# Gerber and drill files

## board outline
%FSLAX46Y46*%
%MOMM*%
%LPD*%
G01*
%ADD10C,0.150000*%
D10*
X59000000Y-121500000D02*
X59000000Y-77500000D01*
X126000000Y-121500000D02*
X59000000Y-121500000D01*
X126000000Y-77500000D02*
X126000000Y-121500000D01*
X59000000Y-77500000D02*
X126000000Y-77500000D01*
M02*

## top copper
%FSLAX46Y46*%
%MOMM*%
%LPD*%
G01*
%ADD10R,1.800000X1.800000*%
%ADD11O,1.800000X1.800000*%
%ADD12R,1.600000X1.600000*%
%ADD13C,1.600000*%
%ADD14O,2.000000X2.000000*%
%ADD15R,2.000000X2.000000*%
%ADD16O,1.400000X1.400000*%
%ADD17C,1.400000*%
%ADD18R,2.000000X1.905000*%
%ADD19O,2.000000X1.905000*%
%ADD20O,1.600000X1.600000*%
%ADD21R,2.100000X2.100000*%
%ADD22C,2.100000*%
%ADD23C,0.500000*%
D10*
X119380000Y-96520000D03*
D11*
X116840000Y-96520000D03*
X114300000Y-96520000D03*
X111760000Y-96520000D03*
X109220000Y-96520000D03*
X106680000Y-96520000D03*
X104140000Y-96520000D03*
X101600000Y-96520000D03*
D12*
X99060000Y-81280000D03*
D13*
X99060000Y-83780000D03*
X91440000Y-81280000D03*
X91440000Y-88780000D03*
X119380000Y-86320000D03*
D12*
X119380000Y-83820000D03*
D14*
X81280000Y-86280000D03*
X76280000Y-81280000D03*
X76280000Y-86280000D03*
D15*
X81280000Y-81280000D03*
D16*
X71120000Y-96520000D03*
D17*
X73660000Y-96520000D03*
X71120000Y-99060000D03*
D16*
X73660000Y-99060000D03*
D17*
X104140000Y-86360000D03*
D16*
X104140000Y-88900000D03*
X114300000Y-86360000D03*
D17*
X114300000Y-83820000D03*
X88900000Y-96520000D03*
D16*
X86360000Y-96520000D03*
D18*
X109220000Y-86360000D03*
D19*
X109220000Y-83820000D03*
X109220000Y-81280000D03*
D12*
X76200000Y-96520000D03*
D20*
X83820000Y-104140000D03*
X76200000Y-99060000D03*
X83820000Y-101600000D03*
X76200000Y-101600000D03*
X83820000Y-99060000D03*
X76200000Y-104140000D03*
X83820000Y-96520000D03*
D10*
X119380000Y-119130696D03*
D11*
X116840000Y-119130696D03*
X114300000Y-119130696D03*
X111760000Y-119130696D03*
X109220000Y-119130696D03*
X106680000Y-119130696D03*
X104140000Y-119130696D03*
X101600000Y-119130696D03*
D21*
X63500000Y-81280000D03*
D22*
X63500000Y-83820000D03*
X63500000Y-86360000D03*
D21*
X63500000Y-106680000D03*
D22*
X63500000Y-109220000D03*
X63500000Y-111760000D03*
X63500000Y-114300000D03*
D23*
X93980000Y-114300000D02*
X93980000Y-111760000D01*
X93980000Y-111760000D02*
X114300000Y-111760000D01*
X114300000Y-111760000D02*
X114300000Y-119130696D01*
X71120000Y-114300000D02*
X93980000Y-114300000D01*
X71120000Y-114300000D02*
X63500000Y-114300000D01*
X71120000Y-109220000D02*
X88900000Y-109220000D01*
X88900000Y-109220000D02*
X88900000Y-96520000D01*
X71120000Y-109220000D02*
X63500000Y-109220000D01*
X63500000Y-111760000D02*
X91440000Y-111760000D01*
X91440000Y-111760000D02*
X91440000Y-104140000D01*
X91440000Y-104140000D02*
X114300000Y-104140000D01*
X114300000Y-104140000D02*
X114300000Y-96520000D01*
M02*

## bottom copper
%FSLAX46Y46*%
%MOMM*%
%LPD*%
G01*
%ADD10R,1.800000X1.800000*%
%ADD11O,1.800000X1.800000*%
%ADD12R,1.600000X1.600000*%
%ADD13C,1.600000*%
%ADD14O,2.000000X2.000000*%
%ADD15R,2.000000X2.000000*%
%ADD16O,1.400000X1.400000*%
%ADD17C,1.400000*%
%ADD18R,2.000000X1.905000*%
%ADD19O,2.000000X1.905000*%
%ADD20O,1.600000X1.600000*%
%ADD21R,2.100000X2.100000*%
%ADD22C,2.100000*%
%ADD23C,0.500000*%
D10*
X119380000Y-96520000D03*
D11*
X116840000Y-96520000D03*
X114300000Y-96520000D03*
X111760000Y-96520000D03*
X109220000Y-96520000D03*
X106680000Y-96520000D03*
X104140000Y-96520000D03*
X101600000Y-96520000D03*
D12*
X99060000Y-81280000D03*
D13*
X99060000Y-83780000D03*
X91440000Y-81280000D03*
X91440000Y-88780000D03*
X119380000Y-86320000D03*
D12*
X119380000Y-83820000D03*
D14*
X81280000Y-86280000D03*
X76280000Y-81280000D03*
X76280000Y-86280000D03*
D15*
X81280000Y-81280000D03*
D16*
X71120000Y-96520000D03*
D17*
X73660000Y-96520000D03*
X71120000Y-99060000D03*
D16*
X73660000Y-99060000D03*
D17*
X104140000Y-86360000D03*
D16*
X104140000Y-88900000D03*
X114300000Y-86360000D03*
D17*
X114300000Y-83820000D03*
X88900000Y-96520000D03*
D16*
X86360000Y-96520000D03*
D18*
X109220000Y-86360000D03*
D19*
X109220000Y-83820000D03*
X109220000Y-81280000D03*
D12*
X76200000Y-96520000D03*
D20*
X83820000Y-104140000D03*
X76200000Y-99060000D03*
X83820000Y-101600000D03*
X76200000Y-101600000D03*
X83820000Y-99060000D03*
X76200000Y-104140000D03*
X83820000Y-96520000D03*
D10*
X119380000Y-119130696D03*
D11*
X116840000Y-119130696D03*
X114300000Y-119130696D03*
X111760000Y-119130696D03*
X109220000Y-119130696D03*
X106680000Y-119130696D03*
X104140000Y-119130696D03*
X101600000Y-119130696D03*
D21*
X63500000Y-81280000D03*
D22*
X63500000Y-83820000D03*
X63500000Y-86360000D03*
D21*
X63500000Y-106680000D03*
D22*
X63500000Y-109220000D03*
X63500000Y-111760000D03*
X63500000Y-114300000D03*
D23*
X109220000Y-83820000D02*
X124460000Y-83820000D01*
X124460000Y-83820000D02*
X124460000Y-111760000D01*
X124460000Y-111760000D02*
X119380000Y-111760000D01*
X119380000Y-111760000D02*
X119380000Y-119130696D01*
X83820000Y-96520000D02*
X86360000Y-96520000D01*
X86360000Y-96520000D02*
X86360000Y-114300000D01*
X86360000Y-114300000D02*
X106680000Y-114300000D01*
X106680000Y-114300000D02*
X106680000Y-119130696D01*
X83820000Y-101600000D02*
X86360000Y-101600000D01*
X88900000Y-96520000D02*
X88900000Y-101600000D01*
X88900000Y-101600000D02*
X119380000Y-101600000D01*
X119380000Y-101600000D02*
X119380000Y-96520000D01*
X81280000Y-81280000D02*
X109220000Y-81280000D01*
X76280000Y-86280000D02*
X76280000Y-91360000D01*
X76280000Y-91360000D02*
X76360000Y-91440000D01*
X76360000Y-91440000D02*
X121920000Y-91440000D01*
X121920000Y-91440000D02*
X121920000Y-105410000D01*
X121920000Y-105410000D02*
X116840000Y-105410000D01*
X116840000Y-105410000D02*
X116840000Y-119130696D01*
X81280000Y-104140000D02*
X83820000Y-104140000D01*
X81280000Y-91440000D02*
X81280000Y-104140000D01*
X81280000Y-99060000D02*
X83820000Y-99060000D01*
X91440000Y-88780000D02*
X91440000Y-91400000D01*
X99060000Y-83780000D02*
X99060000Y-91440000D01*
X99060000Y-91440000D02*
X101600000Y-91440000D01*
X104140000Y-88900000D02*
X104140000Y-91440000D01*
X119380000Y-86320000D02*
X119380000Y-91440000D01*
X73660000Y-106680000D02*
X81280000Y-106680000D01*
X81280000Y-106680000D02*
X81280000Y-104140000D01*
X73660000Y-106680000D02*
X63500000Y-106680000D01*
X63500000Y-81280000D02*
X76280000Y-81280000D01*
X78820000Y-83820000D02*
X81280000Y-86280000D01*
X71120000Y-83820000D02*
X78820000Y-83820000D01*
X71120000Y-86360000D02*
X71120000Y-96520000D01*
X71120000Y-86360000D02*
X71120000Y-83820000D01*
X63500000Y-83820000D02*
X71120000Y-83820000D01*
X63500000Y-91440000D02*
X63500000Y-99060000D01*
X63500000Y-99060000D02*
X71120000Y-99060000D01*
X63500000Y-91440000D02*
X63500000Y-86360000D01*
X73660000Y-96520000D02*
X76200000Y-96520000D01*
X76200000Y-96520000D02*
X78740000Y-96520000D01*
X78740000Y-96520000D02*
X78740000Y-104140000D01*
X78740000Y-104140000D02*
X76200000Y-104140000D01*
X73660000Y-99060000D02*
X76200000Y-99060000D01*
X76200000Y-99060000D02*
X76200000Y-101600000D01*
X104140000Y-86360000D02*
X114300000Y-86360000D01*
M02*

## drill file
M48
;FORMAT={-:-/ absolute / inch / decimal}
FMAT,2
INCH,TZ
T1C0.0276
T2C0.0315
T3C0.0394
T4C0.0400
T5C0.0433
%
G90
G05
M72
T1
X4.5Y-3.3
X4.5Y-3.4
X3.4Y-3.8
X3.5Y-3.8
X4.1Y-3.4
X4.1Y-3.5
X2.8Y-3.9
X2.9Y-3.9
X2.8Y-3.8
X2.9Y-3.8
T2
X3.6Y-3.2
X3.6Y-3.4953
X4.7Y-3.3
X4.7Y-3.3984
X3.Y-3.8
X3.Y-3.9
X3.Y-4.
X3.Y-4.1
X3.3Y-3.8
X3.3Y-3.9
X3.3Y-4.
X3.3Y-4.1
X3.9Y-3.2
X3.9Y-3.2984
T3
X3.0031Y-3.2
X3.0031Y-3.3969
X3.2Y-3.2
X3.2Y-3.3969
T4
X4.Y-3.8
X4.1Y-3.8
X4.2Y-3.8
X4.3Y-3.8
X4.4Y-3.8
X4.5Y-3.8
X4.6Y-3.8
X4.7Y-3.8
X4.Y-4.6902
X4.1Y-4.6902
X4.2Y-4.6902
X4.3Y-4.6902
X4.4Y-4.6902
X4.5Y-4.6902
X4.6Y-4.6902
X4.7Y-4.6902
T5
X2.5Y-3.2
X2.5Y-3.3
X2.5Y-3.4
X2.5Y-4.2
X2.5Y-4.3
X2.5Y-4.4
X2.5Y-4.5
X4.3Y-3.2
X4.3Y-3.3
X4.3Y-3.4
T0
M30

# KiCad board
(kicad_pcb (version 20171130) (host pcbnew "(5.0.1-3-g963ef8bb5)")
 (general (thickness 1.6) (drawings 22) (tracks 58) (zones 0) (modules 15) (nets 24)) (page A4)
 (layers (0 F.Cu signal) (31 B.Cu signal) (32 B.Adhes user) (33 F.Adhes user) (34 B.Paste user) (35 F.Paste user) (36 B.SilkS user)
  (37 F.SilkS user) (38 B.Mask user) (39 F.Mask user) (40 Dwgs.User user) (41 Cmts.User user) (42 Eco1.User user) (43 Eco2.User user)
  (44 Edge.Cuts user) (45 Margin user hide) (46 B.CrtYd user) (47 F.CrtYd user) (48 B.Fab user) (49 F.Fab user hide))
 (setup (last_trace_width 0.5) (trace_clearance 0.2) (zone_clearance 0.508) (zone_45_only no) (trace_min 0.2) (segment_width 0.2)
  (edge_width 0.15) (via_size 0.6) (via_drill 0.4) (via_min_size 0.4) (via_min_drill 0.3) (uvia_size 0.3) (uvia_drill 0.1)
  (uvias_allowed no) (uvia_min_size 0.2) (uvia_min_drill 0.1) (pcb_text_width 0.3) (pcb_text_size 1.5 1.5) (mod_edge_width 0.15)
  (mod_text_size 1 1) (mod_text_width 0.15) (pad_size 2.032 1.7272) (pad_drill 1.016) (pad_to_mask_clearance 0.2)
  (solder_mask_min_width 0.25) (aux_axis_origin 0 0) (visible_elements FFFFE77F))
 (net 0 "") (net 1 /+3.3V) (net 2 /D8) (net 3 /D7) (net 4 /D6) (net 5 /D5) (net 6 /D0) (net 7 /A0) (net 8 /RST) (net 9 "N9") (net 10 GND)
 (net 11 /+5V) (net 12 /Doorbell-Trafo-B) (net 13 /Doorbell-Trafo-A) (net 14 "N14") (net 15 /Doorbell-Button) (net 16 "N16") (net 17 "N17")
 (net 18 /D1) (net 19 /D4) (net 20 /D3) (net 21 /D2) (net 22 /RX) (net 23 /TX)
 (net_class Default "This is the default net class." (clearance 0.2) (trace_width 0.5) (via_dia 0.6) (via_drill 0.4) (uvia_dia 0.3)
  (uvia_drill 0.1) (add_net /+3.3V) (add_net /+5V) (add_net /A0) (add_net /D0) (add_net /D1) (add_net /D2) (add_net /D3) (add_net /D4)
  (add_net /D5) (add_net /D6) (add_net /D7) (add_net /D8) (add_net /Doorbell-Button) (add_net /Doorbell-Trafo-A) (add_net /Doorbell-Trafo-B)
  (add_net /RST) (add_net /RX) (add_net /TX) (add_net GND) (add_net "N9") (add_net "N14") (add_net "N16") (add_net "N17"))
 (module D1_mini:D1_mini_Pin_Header (layer F.Cu) (at 119.38 96.52 270)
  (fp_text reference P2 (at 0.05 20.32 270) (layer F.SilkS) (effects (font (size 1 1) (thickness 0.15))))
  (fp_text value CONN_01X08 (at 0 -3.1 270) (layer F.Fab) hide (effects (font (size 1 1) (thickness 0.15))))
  (pad 1 thru_hole rect (at 0 0 270) (size 1.8 1.8) (drill 1.016) (layers *.Cu *.Mask F.SilkS) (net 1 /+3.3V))
  (pad 2 thru_hole oval (at 0 2.54 270) (size 1.8 1.8) (drill 1.016) (layers *.Cu *.Mask F.SilkS) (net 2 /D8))
  (pad 3 thru_hole oval (at 0 5.08 270) (size 1.8 1.8) (drill 1.016) (layers *.Cu *.Mask F.SilkS) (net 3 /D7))
  (pad 4 thru_hole oval (at 0 7.62 270) (size 1.8 1.8) (drill 1.016) (layers *.Cu *.Mask F.SilkS) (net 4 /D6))
  (pad 5 thru_hole oval (at 0 10.16 270) (size 1.8 1.8) (drill 1.016) (layers *.Cu *.Mask F.SilkS) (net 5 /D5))
  (pad 6 thru_hole oval (at 0 12.7 270) (size 1.8 1.8) (drill 1.016) (layers *.Cu *.Mask F.SilkS) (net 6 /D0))
  (pad 7 thru_hole oval (at 0 15.24 270) (size 1.8 1.8) (drill 1.016) (layers *.Cu *.Mask F.SilkS) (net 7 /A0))
  (pad 8 thru_hole oval (at 0 17.78 270) (size 1.8 1.8) (drill 1.016) (layers *.Cu *.Mask F.SilkS) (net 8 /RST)))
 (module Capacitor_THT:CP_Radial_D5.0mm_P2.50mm (layer F.Cu) (at 99.06 81.28 270)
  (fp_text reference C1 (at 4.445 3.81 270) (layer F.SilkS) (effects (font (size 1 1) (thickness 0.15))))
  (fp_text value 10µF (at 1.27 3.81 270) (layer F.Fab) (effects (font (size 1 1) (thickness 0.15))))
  (pad 1 thru_hole rect (at 0 0 270) (size 1.6 1.6) (drill 0.8) (layers *.Cu *.Mask) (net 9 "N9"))
  (pad 2 thru_hole circle (at 2.5 0 270) (size 1.6 1.6) (drill 0.8) (layers *.Cu *.Mask) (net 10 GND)))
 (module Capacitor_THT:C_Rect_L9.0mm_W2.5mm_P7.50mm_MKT (layer F.Cu) (at 91.44 81.28 270)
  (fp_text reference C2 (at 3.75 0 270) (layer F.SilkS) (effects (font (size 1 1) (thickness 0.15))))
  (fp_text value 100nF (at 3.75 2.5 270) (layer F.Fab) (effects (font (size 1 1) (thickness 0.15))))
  (pad 1 thru_hole circle (at 0 0 270) (size 1.6 1.6) (drill 0.8) (layers *.Cu *.Mask) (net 9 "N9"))
  (pad 2 thru_hole circle (at 7.5 0 270) (size 1.6 1.6) (drill 0.8) (layers *.Cu *.Mask) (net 10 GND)))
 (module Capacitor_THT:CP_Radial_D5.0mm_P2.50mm (layer F.Cu) (at 119.38 83.82 270)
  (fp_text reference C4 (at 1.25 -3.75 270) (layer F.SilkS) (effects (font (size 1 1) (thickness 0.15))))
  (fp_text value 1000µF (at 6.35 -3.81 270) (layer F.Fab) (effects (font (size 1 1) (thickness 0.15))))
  (pad 2 thru_hole circle (at 2.5 0 270) (size 1.6 1.6) (drill 0.8) (layers *.Cu *.Mask) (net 10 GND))
  (pad 1 thru_hole rect (at 0 0 270) (size 1.6 1.6) (drill 0.8) (layers *.Cu *.Mask) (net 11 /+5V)))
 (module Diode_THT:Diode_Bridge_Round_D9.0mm (layer F.Cu) (at 81.28 81.28 270)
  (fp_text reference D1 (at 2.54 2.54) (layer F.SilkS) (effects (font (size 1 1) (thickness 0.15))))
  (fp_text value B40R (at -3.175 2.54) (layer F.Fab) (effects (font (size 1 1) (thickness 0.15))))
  (pad 4 thru_hole oval (at 5 0 270) (size 2 2) (drill 1) (layers *.Cu *.Mask) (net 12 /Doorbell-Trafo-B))
  (pad 2 thru_hole oval (at 0 5 270) (size 2 2) (drill 1) (layers *.Cu *.Mask) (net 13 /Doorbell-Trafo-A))
  (pad 3 thru_hole oval (at 5 5 270) (size 2 2) (drill 1) (layers *.Cu *.Mask) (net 10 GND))
  (pad 1 thru_hole rect (at 0 0 270) (size 2 2) (drill 1) (layers *.Cu *.Mask) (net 9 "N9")))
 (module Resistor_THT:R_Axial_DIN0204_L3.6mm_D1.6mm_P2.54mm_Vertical (layer F.Cu) (at 73.66 96.52 180)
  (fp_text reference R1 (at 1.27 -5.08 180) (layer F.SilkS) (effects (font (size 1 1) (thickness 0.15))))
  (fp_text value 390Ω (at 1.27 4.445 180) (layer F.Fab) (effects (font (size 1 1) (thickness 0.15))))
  (pad 2 thru_hole oval (at 2.54 0 180) (size 1.4 1.4) (drill 0.7) (layers *.Cu *.Mask) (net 12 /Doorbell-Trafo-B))
  (pad 1 thru_hole circle (at 0 0 180) (size 1.4 1.4) (drill 0.7) (layers *.Cu *.Mask) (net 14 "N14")))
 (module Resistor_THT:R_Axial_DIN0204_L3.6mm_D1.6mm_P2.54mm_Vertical (layer F.Cu) (at 71.12 99.06)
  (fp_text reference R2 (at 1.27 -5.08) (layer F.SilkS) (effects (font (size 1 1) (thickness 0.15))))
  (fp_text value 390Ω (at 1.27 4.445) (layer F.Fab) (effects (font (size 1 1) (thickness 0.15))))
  (pad 1 thru_hole circle (at 0 0) (size 1.4 1.4) (drill 0.7) (layers *.Cu *.Mask) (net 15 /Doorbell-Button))
  (pad 2 thru_hole oval (at 2.54 0) (size 1.4 1.4) (drill 0.7) (layers *.Cu *.Mask) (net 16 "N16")))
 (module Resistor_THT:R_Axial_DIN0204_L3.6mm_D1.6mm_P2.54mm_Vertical (layer F.Cu) (at 104.14 86.36 270)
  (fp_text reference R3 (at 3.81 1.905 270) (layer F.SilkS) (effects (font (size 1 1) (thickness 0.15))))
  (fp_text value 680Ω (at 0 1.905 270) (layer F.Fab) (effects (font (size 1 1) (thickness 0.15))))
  (pad 1 thru_hole circle (at 0 0 270) (size 1.4 1.4) (drill 0.7) (layers *.Cu *.Mask) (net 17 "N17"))
  (pad 2 thru_hole oval (at 2.54 0 270) (size 1.4 1.4) (drill 0.7) (layers *.Cu *.Mask) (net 10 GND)))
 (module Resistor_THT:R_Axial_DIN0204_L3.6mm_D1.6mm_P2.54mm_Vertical (layer F.Cu) (at 114.3 83.82 270)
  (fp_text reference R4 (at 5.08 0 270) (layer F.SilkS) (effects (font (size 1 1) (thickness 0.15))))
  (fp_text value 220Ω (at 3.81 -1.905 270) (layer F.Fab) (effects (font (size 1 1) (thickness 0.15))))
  (pad 2 thru_hole oval (at 2.54 0 270) (size 1.4 1.4) (drill 0.7) (layers *.Cu *.Mask) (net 17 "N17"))
  (pad 1 thru_hole circle (at 0 0 270) (size 1.4 1.4) (drill 0.7) (layers *.Cu *.Mask) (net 11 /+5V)))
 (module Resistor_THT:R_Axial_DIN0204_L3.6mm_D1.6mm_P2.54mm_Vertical (layer F.Cu) (at 88.9 96.52 180)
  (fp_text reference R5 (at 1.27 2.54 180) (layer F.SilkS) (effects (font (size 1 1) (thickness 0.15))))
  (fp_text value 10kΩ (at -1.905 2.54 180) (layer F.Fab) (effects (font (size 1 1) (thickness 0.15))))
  (pad 1 thru_hole circle (at 0 0 180) (size 1.4 1.4) (drill 0.7) (layers *.Cu *.Mask) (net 1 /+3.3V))
  (pad 2 thru_hole oval (at 2.54 0 180) (size 1.4 1.4) (drill 0.7) (layers *.Cu *.Mask) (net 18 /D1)))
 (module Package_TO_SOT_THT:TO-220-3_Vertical (layer F.Cu) (at 109.22 86.36 90)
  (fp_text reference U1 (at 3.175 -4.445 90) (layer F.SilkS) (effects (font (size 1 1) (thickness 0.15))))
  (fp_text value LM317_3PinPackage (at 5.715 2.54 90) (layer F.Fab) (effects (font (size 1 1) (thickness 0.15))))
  (pad 1 thru_hole rect (at 0 0 90) (size 1.905 2) (drill 1.1) (layers *.Cu *.Mask) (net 17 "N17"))
  (pad 2 thru_hole oval (at 2.54 0 90) (size 1.905 2) (drill 1.1) (layers *.Cu *.Mask) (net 11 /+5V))
  (pad 3 thru_hole oval (at 5.08 0 90) (size 1.905 2) (drill 1.1) (layers *.Cu *.Mask) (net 9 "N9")))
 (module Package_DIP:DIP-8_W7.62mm (layer F.Cu) (at 76.2 96.52)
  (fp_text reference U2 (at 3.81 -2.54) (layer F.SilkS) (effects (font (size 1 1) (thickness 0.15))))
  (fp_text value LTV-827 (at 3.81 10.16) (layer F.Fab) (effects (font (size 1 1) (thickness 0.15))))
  (pad 1 thru_hole rect (at 0 0) (size 1.6 1.6) (drill 0.8) (layers *.Cu *.Mask) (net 14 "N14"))
  (pad 5 thru_hole oval (at 7.62 7.62) (size 1.6 1.6) (drill 0.8) (layers *.Cu *.Mask) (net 10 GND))
  (pad 2 thru_hole oval (at 0 2.54) (size 1.6 1.6) (drill 0.8) (layers *.Cu *.Mask) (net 16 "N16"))
  (pad 6 thru_hole oval (at 7.62 5.08) (size 1.6 1.6) (drill 0.8) (layers *.Cu *.Mask) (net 18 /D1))
  (pad 3 thru_hole oval (at 0 5.08) (size 1.6 1.6) (drill 0.8) (layers *.Cu *.Mask) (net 16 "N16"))
  (pad 7 thru_hole oval (at 7.62 2.54) (size 1.6 1.6) (drill 0.8) (layers *.Cu *.Mask) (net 10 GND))
  (pad 4 thru_hole oval (at 0 7.62) (size 1.6 1.6) (drill 0.8) (layers *.Cu *.Mask) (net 14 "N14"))
  (pad 8 thru_hole oval (at 7.62 0) (size 1.6 1.6) (drill 0.8) (layers *.Cu *.Mask) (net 18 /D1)))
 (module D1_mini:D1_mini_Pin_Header (layer F.Cu) (at 119.38 119.130696 270)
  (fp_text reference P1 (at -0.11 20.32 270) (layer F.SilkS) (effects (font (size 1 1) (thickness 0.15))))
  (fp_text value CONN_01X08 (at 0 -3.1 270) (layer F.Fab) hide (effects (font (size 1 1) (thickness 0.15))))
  (pad 1 thru_hole rect (at 0 0 270) (size 1.8 1.8) (drill 1.016) (layers *.Cu *.Mask F.SilkS) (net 11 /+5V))
  (pad 2 thru_hole oval (at 0 2.54 270) (size 1.8 1.8) (drill 1.016) (layers *.Cu *.Mask F.SilkS) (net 10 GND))
  (pad 3 thru_hole oval (at 0 5.08 270) (size 1.8 1.8) (drill 1.016) (layers *.Cu *.Mask F.SilkS) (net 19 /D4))
  (pad 4 thru_hole oval (at 0 7.62 270) (size 1.8 1.8) (drill 1.016) (layers *.Cu *.Mask F.SilkS) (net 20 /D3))
  (pad 5 thru_hole oval (at 0 10.16 270) (size 1.8 1.8) (drill 1.016) (layers *.Cu *.Mask F.SilkS) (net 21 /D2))
  (pad 6 thru_hole oval (at 0 12.7 270) (size 1.8 1.8) (drill 1.016) (layers *.Cu *.Mask F.SilkS) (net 18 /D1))
  (pad 7 thru_hole oval (at 0 15.24 270) (size 1.8 1.8) (drill 1.016) (layers *.Cu *.Mask F.SilkS) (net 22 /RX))
  (pad 8 thru_hole oval (at 0 17.78 270) (size 1.8 1.8) (drill 1.016) (layers *.Cu *.Mask F.SilkS) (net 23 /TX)))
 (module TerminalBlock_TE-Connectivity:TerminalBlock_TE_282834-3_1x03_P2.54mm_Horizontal (layer F.Cu) (at 63.5 81.28 270)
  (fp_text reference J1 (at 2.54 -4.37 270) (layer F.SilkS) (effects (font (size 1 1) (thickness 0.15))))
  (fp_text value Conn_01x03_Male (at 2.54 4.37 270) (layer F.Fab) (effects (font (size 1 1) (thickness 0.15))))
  (pad 1 thru_hole rect (at 0 0 270) (size 2.1 2.1) (drill 1.1) (layers *.Cu *.Mask) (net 13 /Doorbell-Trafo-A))
  (pad 2 thru_hole circle (at 2.54 0 270) (size 2.1 2.1) (drill 1.1) (layers *.Cu *.Mask) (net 12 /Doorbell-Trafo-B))
  (pad 3 thru_hole circle (at 5.08 0 270) (size 2.1 2.1) (drill 1.1) (layers *.Cu *.Mask) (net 15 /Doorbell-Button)))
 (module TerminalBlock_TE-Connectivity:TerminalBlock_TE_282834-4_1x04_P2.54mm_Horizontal (layer F.Cu) (at 63.5 106.68 270)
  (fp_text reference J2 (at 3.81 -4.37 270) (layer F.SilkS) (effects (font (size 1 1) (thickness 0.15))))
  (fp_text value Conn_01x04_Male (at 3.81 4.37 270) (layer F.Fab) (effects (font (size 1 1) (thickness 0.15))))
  (pad 1 thru_hole rect (at 0 0 270) (size 2.1 2.1) (drill 1.1) (layers *.Cu *.Mask) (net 10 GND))
  (pad 2 thru_hole circle (at 2.54 0 270) (size 2.1 2.1) (drill 1.1) (layers *.Cu *.Mask) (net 1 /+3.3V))
  (pad 3 thru_hole circle (at 5.08 0 270) (size 2.1 2.1) (drill 1.1) (layers *.Cu *.Mask) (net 3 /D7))
  (pad 4 thru_hole circle (at 7.62 0 270) (size 2.1 2.1) (drill 1.1) (layers *.Cu *.Mask) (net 19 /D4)))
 (gr_line (start 59 121.5) (end 59 77.5) (layer Edge.Cuts) (width 0.15))
 (gr_line (start 126 121.5) (end 59 121.5) (layer Edge.Cuts) (width 0.15))
 (gr_line (start 126 77.5) (end 126 121.5) (layer Edge.Cuts) (width 0.15))
 (gr_line (start 59 77.5) (end 126 77.5) (layer Edge.Cuts) (width 0.15))
 (segment (start 109.22 83.82) (end 124.46 83.82) (width 0.5) (layer B.Cu) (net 11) (status 10))
 (segment (start 124.46 83.82) (end 124.46 111.76) (width 0.5) (layer B.Cu) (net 11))
 (segment (start 124.46 111.76) (end 119.38 111.76) (width 0.5) (layer B.Cu) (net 11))
 (segment (start 119.38 111.76) (end 119.38 119.130696) (width 0.5) (layer B.Cu) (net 11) (status 20))
 (segment (start 93.98 114.3) (end 93.98 111.76) (width 0.5) (layer F.Cu) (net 19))
 (segment (start 93.98 111.76) (end 114.3 111.76) (width 0.5) (layer F.Cu) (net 19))
 (segment (start 114.3 111.76) (end 114.3 119.130696) (width 0.5) (layer F.Cu) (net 19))
 (segment (start 71.12 114.3) (end 93.98 114.3) (width 0.5) (layer F.Cu) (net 19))
 (segment (start 71.12 114.3) (end 63.5 114.3) (width 0.5) (layer F.Cu) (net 19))
 (segment (start 83.82 96.52) (end 86.36 96.52) (width 0.5) (layer B.Cu) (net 18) (status 30))
 (segment (start 86.36 96.52) (end 86.36 114.3) (width 0.5) (layer B.Cu) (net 18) (status 10))
 (segment (start 86.36 114.3) (end 106.68 114.3) (width 0.5) (layer B.Cu) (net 18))
 (segment (start 106.68 114.3) (end 106.68 119.130696) (width 0.5) (layer B.Cu) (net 18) (status 20))
 (segment (start 83.82 101.6) (end 86.36 101.6) (width 0.5) (layer B.Cu) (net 18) (status 10))
 (segment (start 88.9 96.52) (end 88.9 101.6) (width 0.5) (layer B.Cu) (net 1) (status 10))
 (segment (start 88.9 101.6) (end 119.38 101.6) (width 0.5) (layer B.Cu) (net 1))
 (segment (start 119.38 101.6) (end 119.38 96.52) (width 0.5) (layer B.Cu) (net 1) (status 20))
 (segment (start 71.12 109.22) (end 88.9 109.22) (width 0.5) (layer F.Cu) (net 1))
 (segment (start 88.9 109.22) (end 88.9 96.52) (width 0.5) (layer F.Cu) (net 1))
 (segment (start 71.12 109.22) (end 63.5 109.22) (width 0.5) (layer F.Cu) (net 1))
 (segment (start 63.5 111.76) (end 91.44 111.76) (width 0.5) (layer F.Cu) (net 3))
 (segment (start 91.44 111.76) (end 91.44 104.14) (width 0.5) (layer F.Cu) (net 3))
 (segment (start 91.44 104.14) (end 114.3 104.14) (width 0.5) (layer F.Cu) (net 3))
 (segment (start 114.3 104.14) (end 114.3 96.52) (width 0.5) (layer F.Cu) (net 3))
 (segment (start 81.28 81.28) (end 109.22 81.28) (width 0.5) (layer B.Cu) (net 9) (status 30))
 (segment (start 76.28 86.28) (end 76.28 91.36) (width 0.5) (layer B.Cu) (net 10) (status 10))
 (segment (start 76.28 91.36) (end 76.36 91.44) (width 0.5) (layer B.Cu) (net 10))
 (segment (start 76.36 91.44) (end 121.92 91.44) (width 0.5) (layer B.Cu) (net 10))
 (segment (start 121.92 91.44) (end 121.92 105.41) (width 0.5) (layer B.Cu) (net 10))
 (segment (start 121.92 105.41) (end 116.84 105.41) (width 0.5) (layer B.Cu) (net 10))
 (segment (start 116.84 105.41) (end 116.84 119.130696) (width 0.5) (layer B.Cu) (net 10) (status 20))
 (segment (start 81.28 104.14) (end 83.82 104.14) (width 0.5) (layer B.Cu) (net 10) (status 20))
 (segment (start 81.28 91.44) (end 81.28 104.14) (width 0.5) (layer B.Cu) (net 10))
 (segment (start 81.28 99.06) (end 83.82 99.06) (width 0.5) (layer B.Cu) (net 10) (status 20))
 (segment (start 91.44 88.78) (end 91.44 91.4) (width 0.5) (layer B.Cu) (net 10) (status 10))
 (segment (start 99.06 83.78) (end 99.06 91.44) (width 0.5) (layer B.Cu) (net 10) (status 10))
 (segment (start 99.06 91.44) (end 101.6 91.44) (width 0.5) (layer B.Cu) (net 10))
 (segment (start 104.14 88.9) (end 104.14 91.44) (width 0.5) (layer B.Cu) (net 10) (status 10))
 (segment (start 119.38 86.32) (end 119.38 91.44) (width 0.5) (layer B.Cu) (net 10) (status 10))
 (segment (start 73.66 106.68) (end 81.28 106.68) (width 0.5) (layer B.Cu) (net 10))
 (segment (start 81.28 106.68) (end 81.28 104.14) (width 0.5) (layer B.Cu) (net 10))
 (segment (start 73.66 106.68) (end 63.5 106.68) (width 0.5) (layer B.Cu) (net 10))
 (segment (start 63.5 81.28) (end 76.28 81.28) (width 0.5) (layer B.Cu) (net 13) (status 30))
 (segment (start 78.82 83.82) (end 81.28 86.28) (width 0.5) (layer B.Cu) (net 12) (status 20))
 (segment (start 71.12 83.82) (end 78.82 83.82) (width 0.5) (layer B.Cu) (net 12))
 (segment (start 71.12 86.36) (end 71.12 96.52) (width 0.5) (layer B.Cu) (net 12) (status 20))
 (segment (start 71.12 86.36) (end 71.12 83.82) (width 0.5) (layer B.Cu) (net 12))
 (segment (start 63.5 83.82) (end 71.12 83.82) (width 0.5) (layer B.Cu) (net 12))
 (segment (start 63.5 91.44) (end 63.5 99.06) (width 0.5) (layer B.Cu) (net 15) (status 10))
 (segment (start 63.5 99.06) (end 71.12 99.06) (width 0.5) (layer B.Cu) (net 15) (status 20))
 (segment (start 63.5 91.44) (end 63.5 86.36) (width 0.5) (layer B.Cu) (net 15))
 (segment (start 73.66 96.52) (end 76.2 96.52) (width 0.5) (layer B.Cu) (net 14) (status 30))
 (segment (start 76.2 96.52) (end 78.74 96.52) (width 0.5) (layer B.Cu) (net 14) (status 10))
 (segment (start 78.74 96.52) (end 78.74 104.14) (width 0.5) (layer B.Cu) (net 14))
 (segment (start 78.74 104.14) (end 76.2 104.14) (width 0.5) (layer B.Cu) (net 14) (status 20))
 (segment (start 73.66 99.06) (end 76.2 99.06) (width 0.5) (layer B.Cu) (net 16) (status 30))
 (segment (start 76.2 99.06) (end 76.2 101.6) (width 0.5) (layer B.Cu) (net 16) (status 30))
 (segment (start 104.14 86.36) (end 114.3 86.36) (width 0.5) (layer B.Cu) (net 17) (status 30)))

